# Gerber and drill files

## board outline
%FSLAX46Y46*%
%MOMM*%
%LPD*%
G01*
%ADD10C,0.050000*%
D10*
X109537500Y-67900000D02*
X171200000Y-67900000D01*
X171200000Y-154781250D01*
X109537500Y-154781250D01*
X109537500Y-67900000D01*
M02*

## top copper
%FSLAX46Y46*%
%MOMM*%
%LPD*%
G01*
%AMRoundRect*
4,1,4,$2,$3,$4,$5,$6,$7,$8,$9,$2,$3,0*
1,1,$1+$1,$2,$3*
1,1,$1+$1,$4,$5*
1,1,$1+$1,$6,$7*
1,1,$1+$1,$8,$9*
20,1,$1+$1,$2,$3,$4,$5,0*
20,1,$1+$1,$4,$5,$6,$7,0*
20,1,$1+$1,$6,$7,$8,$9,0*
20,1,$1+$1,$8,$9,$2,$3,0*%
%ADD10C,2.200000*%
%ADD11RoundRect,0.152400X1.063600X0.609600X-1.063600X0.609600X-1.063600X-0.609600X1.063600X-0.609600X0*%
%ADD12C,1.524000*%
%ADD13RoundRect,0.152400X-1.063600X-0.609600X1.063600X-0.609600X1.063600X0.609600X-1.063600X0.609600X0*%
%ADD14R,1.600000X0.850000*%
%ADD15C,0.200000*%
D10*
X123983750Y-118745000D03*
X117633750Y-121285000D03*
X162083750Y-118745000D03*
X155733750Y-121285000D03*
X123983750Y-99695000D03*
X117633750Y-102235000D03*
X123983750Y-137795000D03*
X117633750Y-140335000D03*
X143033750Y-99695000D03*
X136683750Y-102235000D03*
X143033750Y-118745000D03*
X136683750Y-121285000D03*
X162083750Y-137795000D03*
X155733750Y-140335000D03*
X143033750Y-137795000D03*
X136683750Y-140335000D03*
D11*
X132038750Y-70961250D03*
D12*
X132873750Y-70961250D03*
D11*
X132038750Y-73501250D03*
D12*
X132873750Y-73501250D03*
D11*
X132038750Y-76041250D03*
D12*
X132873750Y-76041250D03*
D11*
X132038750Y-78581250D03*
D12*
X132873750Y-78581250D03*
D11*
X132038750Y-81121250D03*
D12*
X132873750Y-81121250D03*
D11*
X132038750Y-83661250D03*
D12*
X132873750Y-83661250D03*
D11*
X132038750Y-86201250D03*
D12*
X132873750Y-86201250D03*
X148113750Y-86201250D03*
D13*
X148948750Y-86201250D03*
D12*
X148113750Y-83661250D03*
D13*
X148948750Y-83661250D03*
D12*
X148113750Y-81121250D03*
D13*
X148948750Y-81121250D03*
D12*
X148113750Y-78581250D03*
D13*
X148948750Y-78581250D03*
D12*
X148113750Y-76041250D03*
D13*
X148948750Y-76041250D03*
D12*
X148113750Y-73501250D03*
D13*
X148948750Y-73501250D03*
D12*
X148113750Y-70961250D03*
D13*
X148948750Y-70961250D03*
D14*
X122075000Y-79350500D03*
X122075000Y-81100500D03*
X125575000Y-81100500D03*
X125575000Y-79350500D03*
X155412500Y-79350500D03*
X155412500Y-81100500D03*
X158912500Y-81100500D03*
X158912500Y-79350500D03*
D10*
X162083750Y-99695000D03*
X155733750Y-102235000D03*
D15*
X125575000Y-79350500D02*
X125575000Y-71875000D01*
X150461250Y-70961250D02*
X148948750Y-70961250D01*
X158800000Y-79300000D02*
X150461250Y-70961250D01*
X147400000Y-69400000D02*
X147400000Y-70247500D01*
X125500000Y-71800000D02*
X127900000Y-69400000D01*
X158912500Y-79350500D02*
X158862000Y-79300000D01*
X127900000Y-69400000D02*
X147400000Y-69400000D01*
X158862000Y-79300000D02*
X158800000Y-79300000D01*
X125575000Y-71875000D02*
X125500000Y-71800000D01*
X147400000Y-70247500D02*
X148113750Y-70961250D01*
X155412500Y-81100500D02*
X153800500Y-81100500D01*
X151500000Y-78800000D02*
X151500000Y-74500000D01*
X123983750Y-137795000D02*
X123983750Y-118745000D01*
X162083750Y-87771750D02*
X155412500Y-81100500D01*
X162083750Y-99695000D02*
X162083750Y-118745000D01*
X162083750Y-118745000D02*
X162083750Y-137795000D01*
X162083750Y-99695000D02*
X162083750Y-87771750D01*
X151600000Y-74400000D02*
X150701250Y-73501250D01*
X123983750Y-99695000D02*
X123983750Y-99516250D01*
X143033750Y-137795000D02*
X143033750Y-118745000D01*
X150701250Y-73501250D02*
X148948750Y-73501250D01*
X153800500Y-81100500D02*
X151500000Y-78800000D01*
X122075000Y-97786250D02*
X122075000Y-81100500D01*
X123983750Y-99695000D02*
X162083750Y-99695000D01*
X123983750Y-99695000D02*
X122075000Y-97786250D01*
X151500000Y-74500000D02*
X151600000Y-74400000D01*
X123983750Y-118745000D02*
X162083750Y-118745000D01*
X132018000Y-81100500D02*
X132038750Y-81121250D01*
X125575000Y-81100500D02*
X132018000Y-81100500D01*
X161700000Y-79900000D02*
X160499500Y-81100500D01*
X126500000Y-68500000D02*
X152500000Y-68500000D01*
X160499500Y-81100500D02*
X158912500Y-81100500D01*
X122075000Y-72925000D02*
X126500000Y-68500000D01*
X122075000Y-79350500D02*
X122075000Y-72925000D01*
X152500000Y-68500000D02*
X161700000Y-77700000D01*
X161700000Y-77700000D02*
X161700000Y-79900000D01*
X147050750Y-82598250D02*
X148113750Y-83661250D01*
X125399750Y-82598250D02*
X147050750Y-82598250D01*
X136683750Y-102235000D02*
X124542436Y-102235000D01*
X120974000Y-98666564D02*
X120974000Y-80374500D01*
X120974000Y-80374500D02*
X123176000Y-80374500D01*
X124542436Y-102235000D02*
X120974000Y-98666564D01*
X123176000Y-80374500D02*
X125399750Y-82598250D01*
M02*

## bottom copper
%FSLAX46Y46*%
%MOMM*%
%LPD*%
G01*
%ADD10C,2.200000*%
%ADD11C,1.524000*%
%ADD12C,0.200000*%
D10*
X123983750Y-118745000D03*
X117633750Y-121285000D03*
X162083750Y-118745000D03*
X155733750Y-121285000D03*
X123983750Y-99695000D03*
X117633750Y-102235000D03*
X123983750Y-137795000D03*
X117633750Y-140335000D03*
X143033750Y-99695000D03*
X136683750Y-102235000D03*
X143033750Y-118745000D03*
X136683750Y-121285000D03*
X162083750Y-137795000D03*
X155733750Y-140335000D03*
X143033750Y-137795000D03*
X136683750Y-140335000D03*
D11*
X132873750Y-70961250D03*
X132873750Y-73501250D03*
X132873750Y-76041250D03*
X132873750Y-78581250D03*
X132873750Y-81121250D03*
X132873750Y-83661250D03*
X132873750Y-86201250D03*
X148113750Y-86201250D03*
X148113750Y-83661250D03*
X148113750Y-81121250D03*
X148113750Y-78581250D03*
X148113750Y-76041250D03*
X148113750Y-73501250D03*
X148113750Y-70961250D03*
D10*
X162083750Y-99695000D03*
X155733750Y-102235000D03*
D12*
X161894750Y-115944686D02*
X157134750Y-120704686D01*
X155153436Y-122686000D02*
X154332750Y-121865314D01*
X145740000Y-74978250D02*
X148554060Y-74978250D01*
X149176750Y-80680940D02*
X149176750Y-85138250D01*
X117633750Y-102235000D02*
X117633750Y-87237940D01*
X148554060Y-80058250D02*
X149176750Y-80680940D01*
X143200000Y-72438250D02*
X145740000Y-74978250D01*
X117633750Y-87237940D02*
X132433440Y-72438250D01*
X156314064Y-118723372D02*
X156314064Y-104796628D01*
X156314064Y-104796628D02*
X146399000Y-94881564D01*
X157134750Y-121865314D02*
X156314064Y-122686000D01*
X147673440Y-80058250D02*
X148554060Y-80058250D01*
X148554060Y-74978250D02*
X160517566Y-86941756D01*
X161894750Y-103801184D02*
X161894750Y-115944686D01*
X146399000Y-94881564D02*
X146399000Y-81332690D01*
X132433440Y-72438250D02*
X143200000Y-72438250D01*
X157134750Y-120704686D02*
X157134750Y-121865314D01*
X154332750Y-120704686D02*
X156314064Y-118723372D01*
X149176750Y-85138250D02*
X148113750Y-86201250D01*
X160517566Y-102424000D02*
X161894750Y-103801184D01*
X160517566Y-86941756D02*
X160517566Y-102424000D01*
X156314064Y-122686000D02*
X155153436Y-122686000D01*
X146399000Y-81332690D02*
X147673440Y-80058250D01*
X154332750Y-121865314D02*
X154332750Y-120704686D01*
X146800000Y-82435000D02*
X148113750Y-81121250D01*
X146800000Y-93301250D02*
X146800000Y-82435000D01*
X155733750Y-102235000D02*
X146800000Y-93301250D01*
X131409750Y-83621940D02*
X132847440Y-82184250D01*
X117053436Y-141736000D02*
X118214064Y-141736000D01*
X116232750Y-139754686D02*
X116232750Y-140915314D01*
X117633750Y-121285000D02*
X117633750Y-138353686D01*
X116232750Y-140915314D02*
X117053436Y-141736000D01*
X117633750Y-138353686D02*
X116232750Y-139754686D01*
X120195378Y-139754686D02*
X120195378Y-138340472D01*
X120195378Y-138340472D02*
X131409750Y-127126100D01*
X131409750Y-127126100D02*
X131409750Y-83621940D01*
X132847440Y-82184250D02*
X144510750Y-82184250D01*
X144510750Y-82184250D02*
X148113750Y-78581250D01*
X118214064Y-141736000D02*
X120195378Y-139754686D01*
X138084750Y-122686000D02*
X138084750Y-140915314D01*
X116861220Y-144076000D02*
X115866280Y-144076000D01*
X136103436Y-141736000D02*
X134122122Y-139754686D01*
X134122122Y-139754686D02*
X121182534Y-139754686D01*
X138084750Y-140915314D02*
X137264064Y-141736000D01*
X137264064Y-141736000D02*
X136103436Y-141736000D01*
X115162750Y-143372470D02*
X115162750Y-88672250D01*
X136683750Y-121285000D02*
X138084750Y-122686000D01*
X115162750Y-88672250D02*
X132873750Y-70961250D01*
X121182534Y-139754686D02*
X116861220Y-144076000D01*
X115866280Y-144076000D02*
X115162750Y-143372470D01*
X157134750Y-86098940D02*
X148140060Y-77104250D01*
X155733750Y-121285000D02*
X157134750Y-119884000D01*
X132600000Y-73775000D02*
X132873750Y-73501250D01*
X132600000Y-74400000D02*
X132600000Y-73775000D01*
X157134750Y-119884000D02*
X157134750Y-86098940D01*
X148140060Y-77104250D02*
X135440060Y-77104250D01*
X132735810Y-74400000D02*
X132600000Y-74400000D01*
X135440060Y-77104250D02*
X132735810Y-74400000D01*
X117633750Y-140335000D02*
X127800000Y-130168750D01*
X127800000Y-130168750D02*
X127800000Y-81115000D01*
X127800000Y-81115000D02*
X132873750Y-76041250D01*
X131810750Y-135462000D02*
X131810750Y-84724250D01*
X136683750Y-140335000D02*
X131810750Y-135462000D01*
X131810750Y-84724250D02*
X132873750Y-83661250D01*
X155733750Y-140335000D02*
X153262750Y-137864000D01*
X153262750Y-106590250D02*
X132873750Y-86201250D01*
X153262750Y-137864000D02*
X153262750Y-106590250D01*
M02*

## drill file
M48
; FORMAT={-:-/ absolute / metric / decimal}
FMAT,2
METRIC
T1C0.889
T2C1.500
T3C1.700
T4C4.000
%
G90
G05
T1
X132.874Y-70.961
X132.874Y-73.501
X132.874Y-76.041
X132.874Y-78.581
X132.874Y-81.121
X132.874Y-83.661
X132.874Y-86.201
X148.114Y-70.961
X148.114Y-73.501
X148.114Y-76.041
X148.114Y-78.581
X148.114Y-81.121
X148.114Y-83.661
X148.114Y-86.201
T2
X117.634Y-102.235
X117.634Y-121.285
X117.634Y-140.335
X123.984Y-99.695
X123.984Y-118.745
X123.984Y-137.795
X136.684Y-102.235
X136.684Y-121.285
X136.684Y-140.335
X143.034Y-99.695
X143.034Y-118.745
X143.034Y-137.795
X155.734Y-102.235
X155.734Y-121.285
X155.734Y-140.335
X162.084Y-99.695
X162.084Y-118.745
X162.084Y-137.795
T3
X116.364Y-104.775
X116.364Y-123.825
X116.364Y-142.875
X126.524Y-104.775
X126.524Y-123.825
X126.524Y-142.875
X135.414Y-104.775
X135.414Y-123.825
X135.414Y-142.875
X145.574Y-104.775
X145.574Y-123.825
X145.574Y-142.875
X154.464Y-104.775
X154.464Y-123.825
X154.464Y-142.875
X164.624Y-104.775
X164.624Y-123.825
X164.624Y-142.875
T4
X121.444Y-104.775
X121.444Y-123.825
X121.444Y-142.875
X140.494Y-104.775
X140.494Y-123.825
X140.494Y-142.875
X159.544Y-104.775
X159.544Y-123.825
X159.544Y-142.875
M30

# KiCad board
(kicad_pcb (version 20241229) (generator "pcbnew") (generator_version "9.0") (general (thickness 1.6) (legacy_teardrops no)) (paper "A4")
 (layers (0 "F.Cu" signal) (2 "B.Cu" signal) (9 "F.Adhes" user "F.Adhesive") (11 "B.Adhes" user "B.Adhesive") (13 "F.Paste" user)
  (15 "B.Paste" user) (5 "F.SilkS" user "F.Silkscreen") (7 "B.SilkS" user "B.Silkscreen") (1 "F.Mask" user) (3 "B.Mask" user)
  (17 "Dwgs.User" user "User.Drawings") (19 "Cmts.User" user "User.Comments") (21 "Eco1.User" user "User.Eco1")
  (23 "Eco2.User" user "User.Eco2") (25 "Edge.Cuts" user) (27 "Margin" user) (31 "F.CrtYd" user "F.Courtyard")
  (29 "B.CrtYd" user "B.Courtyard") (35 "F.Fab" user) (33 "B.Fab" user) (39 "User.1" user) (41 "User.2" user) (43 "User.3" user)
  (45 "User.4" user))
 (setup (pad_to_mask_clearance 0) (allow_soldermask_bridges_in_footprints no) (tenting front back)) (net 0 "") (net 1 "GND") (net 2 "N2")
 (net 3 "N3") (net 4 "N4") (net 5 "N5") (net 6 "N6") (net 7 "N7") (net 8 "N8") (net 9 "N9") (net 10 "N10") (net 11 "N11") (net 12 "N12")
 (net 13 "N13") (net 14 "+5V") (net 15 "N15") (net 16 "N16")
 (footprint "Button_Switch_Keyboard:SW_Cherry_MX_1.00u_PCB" (layer "F.Cu") (at 123.98375 118.745)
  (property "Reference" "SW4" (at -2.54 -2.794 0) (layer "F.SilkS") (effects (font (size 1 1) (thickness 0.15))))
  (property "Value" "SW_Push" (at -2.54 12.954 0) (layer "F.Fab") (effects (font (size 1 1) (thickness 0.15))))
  (pad "" np_thru_hole circle (at -7.62 5.08) (size 1.7 1.7) (drill 1.7) (layers "*.Cu" "*.Mask"))
  (pad "" np_thru_hole circle (at -2.54 5.08) (size 4 4) (drill 4) (layers "*.Cu" "*.Mask"))
  (pad "" np_thru_hole circle (at 2.54 5.08) (size 1.7 1.7) (drill 1.7) (layers "*.Cu" "*.Mask"))
  (pad "1" thru_hole circle (at 0 0) (size 2.2 2.2) (drill 1.5) (layers "*.Cu" "*.Mask") (remove_unused_layers no) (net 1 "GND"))
  (pad "2" thru_hole circle (at -6.35 2.54) (size 2.2 2.2) (drill 1.5) (layers "*.Cu" "*.Mask") (remove_unused_layers no) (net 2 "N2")))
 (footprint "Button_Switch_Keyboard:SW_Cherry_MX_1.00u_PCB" (layer "F.Cu") (at 162.08375 118.745)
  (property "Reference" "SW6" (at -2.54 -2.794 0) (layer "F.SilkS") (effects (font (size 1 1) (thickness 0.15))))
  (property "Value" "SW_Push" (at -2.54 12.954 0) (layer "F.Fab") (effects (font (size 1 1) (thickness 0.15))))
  (pad "" np_thru_hole circle (at -7.62 5.08) (size 1.7 1.7) (drill 1.7) (layers "*.Cu" "*.Mask"))
  (pad "" np_thru_hole circle (at -2.54 5.08) (size 4 4) (drill 4) (layers "*.Cu" "*.Mask"))
  (pad "" np_thru_hole circle (at 2.54 5.08) (size 1.7 1.7) (drill 1.7) (layers "*.Cu" "*.Mask"))
  (pad "1" thru_hole circle (at 0 0) (size 2.2 2.2) (drill 1.5) (layers "*.Cu" "*.Mask") (remove_unused_layers no) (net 1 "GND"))
  (pad "2" thru_hole circle (at -6.35 2.54) (size 2.2 2.2) (drill 1.5) (layers "*.Cu" "*.Mask") (remove_unused_layers no) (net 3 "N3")))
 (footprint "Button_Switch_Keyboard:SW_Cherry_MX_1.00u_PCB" (layer "F.Cu") (at 123.98375 99.695)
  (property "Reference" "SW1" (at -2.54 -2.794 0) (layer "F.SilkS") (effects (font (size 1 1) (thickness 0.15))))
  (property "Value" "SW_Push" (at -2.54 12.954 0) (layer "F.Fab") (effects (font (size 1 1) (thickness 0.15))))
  (pad "" np_thru_hole circle (at -7.62 5.08) (size 1.7 1.7) (drill 1.7) (layers "*.Cu" "*.Mask"))
  (pad "" np_thru_hole circle (at -2.54 5.08) (size 4 4) (drill 4) (layers "*.Cu" "*.Mask"))
  (pad "" np_thru_hole circle (at 2.54 5.08) (size 1.7 1.7) (drill 1.7) (layers "*.Cu" "*.Mask"))
  (pad "1" thru_hole circle (at 0 0) (size 2.2 2.2) (drill 1.5) (layers "*.Cu" "*.Mask") (remove_unused_layers no) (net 1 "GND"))
  (pad "2" thru_hole circle (at -6.35 2.54) (size 2.2 2.2) (drill 1.5) (layers "*.Cu" "*.Mask") (remove_unused_layers no) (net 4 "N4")))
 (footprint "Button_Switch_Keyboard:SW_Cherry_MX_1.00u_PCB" (layer "F.Cu") (at 123.98375 137.795)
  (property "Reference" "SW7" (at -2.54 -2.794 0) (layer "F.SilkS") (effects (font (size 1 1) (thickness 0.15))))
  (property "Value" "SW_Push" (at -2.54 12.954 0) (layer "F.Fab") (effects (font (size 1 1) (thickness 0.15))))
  (pad "" np_thru_hole circle (at -7.62 5.08) (size 1.7 1.7) (drill 1.7) (layers "*.Cu" "*.Mask"))
  (pad "" np_thru_hole circle (at -2.54 5.08) (size 4 4) (drill 4) (layers "*.Cu" "*.Mask"))
  (pad "" np_thru_hole circle (at 2.54 5.08) (size 1.7 1.7) (drill 1.7) (layers "*.Cu" "*.Mask"))
  (pad "1" thru_hole circle (at 0 0) (size 2.2 2.2) (drill 1.5) (layers "*.Cu" "*.Mask") (remove_unused_layers no) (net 1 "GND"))
  (pad "2" thru_hole circle (at -6.35 2.54) (size 2.2 2.2) (drill 1.5) (layers "*.Cu" "*.Mask") (remove_unused_layers no) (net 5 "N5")))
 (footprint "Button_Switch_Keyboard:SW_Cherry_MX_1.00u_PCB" (layer "F.Cu") (at 143.03375 99.695)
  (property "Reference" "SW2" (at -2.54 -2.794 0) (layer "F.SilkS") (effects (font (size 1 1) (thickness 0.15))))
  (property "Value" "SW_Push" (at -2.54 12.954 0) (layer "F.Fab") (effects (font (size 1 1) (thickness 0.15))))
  (pad "" np_thru_hole circle (at -7.62 5.08) (size 1.7 1.7) (drill 1.7) (layers "*.Cu" "*.Mask"))
  (pad "" np_thru_hole circle (at -2.54 5.08) (size 4 4) (drill 4) (layers "*.Cu" "*.Mask"))
  (pad "" np_thru_hole circle (at 2.54 5.08) (size 1.7 1.7) (drill 1.7) (layers "*.Cu" "*.Mask"))
  (pad "1" thru_hole circle (at 0 0) (size 2.2 2.2) (drill 1.5) (layers "*.Cu" "*.Mask") (remove_unused_layers no) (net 1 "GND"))
  (pad "2" thru_hole circle (at -6.35 2.54) (size 2.2 2.2) (drill 1.5) (layers "*.Cu" "*.Mask") (remove_unused_layers no) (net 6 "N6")))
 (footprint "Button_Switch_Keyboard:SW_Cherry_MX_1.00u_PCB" (layer "F.Cu") (at 143.03375 118.745)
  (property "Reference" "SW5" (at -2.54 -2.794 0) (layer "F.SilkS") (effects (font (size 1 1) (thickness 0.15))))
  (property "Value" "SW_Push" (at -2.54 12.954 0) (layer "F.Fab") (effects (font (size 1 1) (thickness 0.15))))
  (pad "" np_thru_hole circle (at -7.62 5.08) (size 1.7 1.7) (drill 1.7) (layers "*.Cu" "*.Mask"))
  (pad "" np_thru_hole circle (at -2.54 5.08) (size 4 4) (drill 4) (layers "*.Cu" "*.Mask"))
  (pad "" np_thru_hole circle (at 2.54 5.08) (size 1.7 1.7) (drill 1.7) (layers "*.Cu" "*.Mask"))
  (pad "1" thru_hole circle (at 0 0) (size 2.2 2.2) (drill 1.5) (layers "*.Cu" "*.Mask") (remove_unused_layers no) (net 1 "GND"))
  (pad "2" thru_hole circle (at -6.35 2.54) (size 2.2 2.2) (drill 1.5) (layers "*.Cu" "*.Mask") (remove_unused_layers no) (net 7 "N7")))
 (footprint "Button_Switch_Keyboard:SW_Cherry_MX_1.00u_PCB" (layer "F.Cu") (at 162.08375 137.795)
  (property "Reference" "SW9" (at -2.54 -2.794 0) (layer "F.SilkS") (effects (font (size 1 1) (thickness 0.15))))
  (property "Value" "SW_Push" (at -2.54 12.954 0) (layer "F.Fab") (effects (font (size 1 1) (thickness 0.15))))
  (pad "" np_thru_hole circle (at -7.62 5.08) (size 1.7 1.7) (drill 1.7) (layers "*.Cu" "*.Mask"))
  (pad "" np_thru_hole circle (at -2.54 5.08) (size 4 4) (drill 4) (layers "*.Cu" "*.Mask"))
  (pad "" np_thru_hole circle (at 2.54 5.08) (size 1.7 1.7) (drill 1.7) (layers "*.Cu" "*.Mask"))
  (pad "1" thru_hole circle (at 0 0) (size 2.2 2.2) (drill 1.5) (layers "*.Cu" "*.Mask") (remove_unused_layers no) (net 1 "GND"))
  (pad "2" thru_hole circle (at -6.35 2.54) (size 2.2 2.2) (drill 1.5) (layers "*.Cu" "*.Mask") (remove_unused_layers no) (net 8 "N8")))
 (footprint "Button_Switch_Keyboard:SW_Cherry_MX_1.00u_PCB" (layer "F.Cu") (at 143.03375 137.795)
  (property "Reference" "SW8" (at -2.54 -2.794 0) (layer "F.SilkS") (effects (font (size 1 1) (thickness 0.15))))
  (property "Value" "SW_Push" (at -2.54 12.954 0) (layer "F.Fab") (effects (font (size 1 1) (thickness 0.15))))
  (pad "" np_thru_hole circle (at -7.62 5.08) (size 1.7 1.7) (drill 1.7) (layers "*.Cu" "*.Mask"))
  (pad "" np_thru_hole circle (at -2.54 5.08) (size 4 4) (drill 4) (layers "*.Cu" "*.Mask"))
  (pad "" np_thru_hole circle (at 2.54 5.08) (size 1.7 1.7) (drill 1.7) (layers "*.Cu" "*.Mask"))
  (pad "1" thru_hole circle (at 0 0) (size 2.2 2.2) (drill 1.5) (layers "*.Cu" "*.Mask") (remove_unused_layers no) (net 1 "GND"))
  (pad "2" thru_hole circle (at -6.35 2.54) (size 2.2 2.2) (drill 1.5) (layers "*.Cu" "*.Mask") (remove_unused_layers no) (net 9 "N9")))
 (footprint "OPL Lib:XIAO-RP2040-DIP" (layer "F.Cu") (at 140.49375 78.58125)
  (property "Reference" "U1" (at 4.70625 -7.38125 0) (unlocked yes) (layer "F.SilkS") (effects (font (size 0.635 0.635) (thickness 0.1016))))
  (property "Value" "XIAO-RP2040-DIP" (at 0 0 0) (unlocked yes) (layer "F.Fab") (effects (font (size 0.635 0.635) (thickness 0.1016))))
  (pad "1" smd roundrect (at -8.455 -7.62 180) (size 2.432 1.524) (layers "F.Cu" "F.Mask") (roundrect_rratio 0.1) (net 7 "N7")
   (thermal_bridge_angle 45))
  (pad "1" thru_hole circle (at -7.62 -7.62 180) (size 1.524 1.524) (drill 0.889) (layers "*.Cu" "*.Mask") (remove_unused_layers no)
   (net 7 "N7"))
  (pad "2" smd roundrect (at -8.455 -5.08 180) (size 2.432 1.524) (layers "F.Cu" "F.Mask") (roundrect_rratio 0.1) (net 3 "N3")
   (thermal_bridge_angle 45))
  (pad "2" thru_hole circle (at -7.62 -5.08 180) (size 1.524 1.524) (drill 0.889) (layers "*.Cu" "*.Mask") (remove_unused_layers no)
   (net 3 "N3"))
  (pad "3" smd roundrect (at -8.455 -2.54 180) (size 2.432 1.524) (layers "F.Cu" "F.Mask") (roundrect_rratio 0.1) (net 5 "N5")
   (thermal_bridge_angle 45))
  (pad "3" thru_hole circle (at -7.62 -2.54 180) (size 1.524 1.524) (drill 0.889) (layers "*.Cu" "*.Mask") (remove_unused_layers no)
   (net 5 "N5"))
  (pad "4" smd roundrect (at -8.455 0 180) (size 2.432 1.524) (layers "F.Cu" "F.Mask") (roundrect_rratio 0.1) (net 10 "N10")
   (thermal_bridge_angle 45))
  (pad "4" thru_hole circle (at -7.62 0 180) (size 1.524 1.524) (drill 0.889) (layers "*.Cu" "*.Mask") (remove_unused_layers no)
   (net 10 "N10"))
  (pad "5" smd roundrect (at -8.455 2.54 180) (size 2.432 1.524) (layers "F.Cu" "F.Mask") (roundrect_rratio 0.1) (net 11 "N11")
   (thermal_bridge_angle 45))
  (pad "5" thru_hole circle (at -7.62 2.54 180) (size 1.524 1.524) (drill 0.889) (layers "*.Cu" "*.Mask") (remove_unused_layers no)
   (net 11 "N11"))
  (pad "6" smd roundrect (at -8.455 5.08 180) (size 2.432 1.524) (layers "F.Cu" "F.Mask") (roundrect_rratio 0.1) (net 9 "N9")
   (thermal_bridge_angle 45))
  (pad "6" thru_hole circle (at -7.62 5.08 180) (size 1.524 1.524) (drill 0.889) (layers "*.Cu" "*.Mask") (remove_unused_layers no)
   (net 9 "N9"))
  (pad "7" smd roundrect (at -8.455 7.62 180) (size 2.432 1.524) (layers "F.Cu" "F.Mask") (roundrect_rratio 0.1) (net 8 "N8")
   (thermal_bridge_angle 45))
  (pad "7" thru_hole circle (at -7.62 7.62 180) (size 1.524 1.524) (drill 0.889) (layers "*.Cu" "*.Mask") (remove_unused_layers no)
   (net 8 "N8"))
  (pad "8" thru_hole circle (at 7.62 7.62) (size 1.524 1.524) (drill 0.889) (layers "*.Cu" "*.Mask") (remove_unused_layers no) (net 4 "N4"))
  (pad "8" smd roundrect (at 8.455 7.62) (size 2.432 1.524) (layers "F.Cu" "F.Mask") (roundrect_rratio 0.1) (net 4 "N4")
   (thermal_bridge_angle 45))
  (pad "9" thru_hole circle (at 7.62 5.08) (size 1.524 1.524) (drill 0.889) (layers "*.Cu" "*.Mask") (remove_unused_layers no) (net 6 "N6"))
  (pad "9" smd roundrect (at 8.455 5.08) (size 2.432 1.524) (layers "F.Cu" "F.Mask") (roundrect_rratio 0.1) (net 6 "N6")
   (thermal_bridge_angle 45))
  (pad "10" thru_hole circle (at 7.62 2.54) (size 1.524 1.524) (drill 0.889) (layers "*.Cu" "*.Mask") (remove_unused_layers no)
   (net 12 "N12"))
  (pad "10" smd roundrect (at 8.455 2.54) (size 2.432 1.524) (layers "F.Cu" "F.Mask") (roundrect_rratio 0.1) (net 12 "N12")
   (thermal_bridge_angle 45))
  (pad "11" thru_hole circle (at 7.62 0) (size 1.524 1.524) (drill 0.889) (layers "*.Cu" "*.Mask") (remove_unused_layers no) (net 2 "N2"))
  (pad "11" smd roundrect (at 8.455 0) (size 2.432 1.524) (layers "F.Cu" "F.Mask") (roundrect_rratio 0.1) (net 2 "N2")
   (thermal_bridge_angle 45))
  (pad "12" thru_hole circle (at 7.62 -2.54) (size 1.524 1.524) (drill 0.889) (layers "*.Cu" "*.Mask") (remove_unused_layers no)
   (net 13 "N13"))
  (pad "12" smd roundrect (at 8.455 -2.54) (size 2.432 1.524) (layers "F.Cu" "F.Mask") (roundrect_rratio 0.1) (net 13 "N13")
   (thermal_bridge_angle 45))
  (pad "13" thru_hole circle (at 7.62 -5.08) (size 1.524 1.524) (drill 0.889) (layers "*.Cu" "*.Mask") (remove_unused_layers no)
   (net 1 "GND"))
  (pad "13" smd roundrect (at 8.455 -5.08) (size 2.432 1.524) (layers "F.Cu" "F.Mask") (roundrect_rratio 0.1) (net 1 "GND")
   (thermal_bridge_angle 45))
  (pad "14" thru_hole circle (at 7.62 -7.62) (size 1.524 1.524) (drill 0.889) (layers "*.Cu" "*.Mask") (remove_unused_layers no)
   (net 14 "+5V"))
  (pad "14" smd roundrect (at 8.455 -7.62) (size 2.432 1.524) (layers "F.Cu" "F.Mask") (roundrect_rratio 0.1) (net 14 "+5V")
   (thermal_bridge_angle 45)))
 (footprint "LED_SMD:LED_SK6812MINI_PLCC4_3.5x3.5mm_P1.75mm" (layer "F.Cu") (at 123.825 80.2255)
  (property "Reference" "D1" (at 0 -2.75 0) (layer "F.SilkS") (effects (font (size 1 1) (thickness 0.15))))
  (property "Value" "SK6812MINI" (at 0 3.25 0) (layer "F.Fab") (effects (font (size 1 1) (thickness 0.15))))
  (pad "1" smd rect (at -1.75 -0.875) (size 1.6 0.85) (layers "F.Cu" "F.Mask" "F.Paste") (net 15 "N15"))
  (pad "2" smd rect (at -1.75 0.875) (size 1.6 0.85) (layers "F.Cu" "F.Mask" "F.Paste") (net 1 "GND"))
  (pad "3" smd rect (at 1.75 0.875) (size 1.6 0.85) (layers "F.Cu" "F.Mask" "F.Paste") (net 11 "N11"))
  (pad "4" smd rect (at 1.75 -0.875) (size 1.6 0.85) (layers "F.Cu" "F.Mask" "F.Paste") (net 14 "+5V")))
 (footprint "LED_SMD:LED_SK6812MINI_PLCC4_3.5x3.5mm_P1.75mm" (layer "F.Cu") (at 157.1625 80.2255)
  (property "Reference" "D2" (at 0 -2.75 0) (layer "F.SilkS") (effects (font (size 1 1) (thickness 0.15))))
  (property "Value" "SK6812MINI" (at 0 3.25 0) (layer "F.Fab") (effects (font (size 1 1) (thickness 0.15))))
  (pad "1" smd rect (at -1.75 -0.875) (size 1.6 0.85) (layers "F.Cu" "F.Mask" "F.Paste") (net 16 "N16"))
  (pad "2" smd rect (at -1.75 0.875) (size 1.6 0.85) (layers "F.Cu" "F.Mask" "F.Paste") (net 1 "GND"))
  (pad "3" smd rect (at 1.75 0.875) (size 1.6 0.85) (layers "F.Cu" "F.Mask" "F.Paste") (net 15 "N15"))
  (pad "4" smd rect (at 1.75 -0.875) (size 1.6 0.85) (layers "F.Cu" "F.Mask" "F.Paste") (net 14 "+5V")))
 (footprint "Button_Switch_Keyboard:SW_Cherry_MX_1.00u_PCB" (layer "F.Cu") (at 162.08375 99.695)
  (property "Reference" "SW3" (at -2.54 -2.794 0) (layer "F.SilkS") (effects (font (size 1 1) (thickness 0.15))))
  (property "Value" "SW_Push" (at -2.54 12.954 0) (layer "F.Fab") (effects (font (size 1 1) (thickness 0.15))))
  (pad "" np_thru_hole circle (at -7.62 5.08) (size 1.7 1.7) (drill 1.7) (layers "*.Cu" "*.Mask"))
  (pad "" np_thru_hole circle (at -2.54 5.08) (size 4 4) (drill 4) (layers "*.Cu" "*.Mask"))
  (pad "" np_thru_hole circle (at 2.54 5.08) (size 1.7 1.7) (drill 1.7) (layers "*.Cu" "*.Mask"))
  (pad "1" thru_hole circle (at 0 0) (size 2.2 2.2) (drill 1.5) (layers "*.Cu" "*.Mask") (remove_unused_layers no) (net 1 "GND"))
  (pad "2" thru_hole circle (at -6.35 2.54) (size 2.2 2.2) (drill 1.5) (layers "*.Cu" "*.Mask") (remove_unused_layers no) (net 12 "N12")))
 (gr_rect (start 109.5375 67.9) (end 171.2 154.78125) (stroke (width 0.05) (type default)) (fill no) (layer "Edge.Cuts"))
 (segment (start 125.575 79.3505) (end 125.575 71.875) (width 0.2) (layer "F.Cu") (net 14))
 (segment (start 150.46125 70.96125) (end 148.94875 70.96125) (width 0.2) (layer "F.Cu") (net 14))
 (segment (start 158.8 79.3) (end 150.46125 70.96125) (width 0.2) (layer "F.Cu") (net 14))
 (segment (start 147.4 69.4) (end 147.4 70.2475) (width 0.2) (layer "F.Cu") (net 14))
 (segment (start 125.5 71.8) (end 127.9 69.4) (width 0.2) (layer "F.Cu") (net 14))
 (segment (start 158.9125 79.3505) (end 158.862 79.3) (width 0.2) (layer "F.Cu") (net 14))
 (segment (start 127.9 69.4) (end 147.4 69.4) (width 0.2) (layer "F.Cu") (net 14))
 (segment (start 158.862 79.3) (end 158.8 79.3) (width 0.2) (layer "F.Cu") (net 14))
 (segment (start 125.575 71.875) (end 125.5 71.8) (width 0.2) (layer "F.Cu") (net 14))
 (segment (start 147.4 70.2475) (end 148.11375 70.96125) (width 0.2) (layer "F.Cu") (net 14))
 (segment (start 155.4125 81.1005) (end 153.8005 81.1005) (width 0.2) (layer "F.Cu") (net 1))
 (segment (start 151.5 78.8) (end 151.5 74.5) (width 0.2) (layer "F.Cu") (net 1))
 (segment (start 123.98375 137.795) (end 123.98375 118.745) (width 0.2) (layer "F.Cu") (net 1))
 (segment (start 162.08375 87.77175) (end 155.4125 81.1005) (width 0.2) (layer "F.Cu") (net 1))
 (segment (start 162.08375 99.695) (end 162.08375 118.745) (width 0.2) (layer "F.Cu") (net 1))
 (segment (start 162.08375 118.745) (end 162.08375 137.795) (width 0.2) (layer "F.Cu") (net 1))
 (segment (start 162.08375 99.695) (end 162.08375 87.77175) (width 0.2) (layer "F.Cu") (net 1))
 (segment (start 151.6 74.4) (end 150.70125 73.50125) (width 0.2) (layer "F.Cu") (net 1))
 (segment (start 123.98375 99.695) (end 123.98375 99.51625) (width 0.2) (layer "F.Cu") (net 1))
 (segment (start 143.03375 137.795) (end 143.03375 118.745) (width 0.2) (layer "F.Cu") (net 1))
 (segment (start 150.70125 73.50125) (end 148.94875 73.50125) (width 0.2) (layer "F.Cu") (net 1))
 (segment (start 153.8005 81.1005) (end 151.5 78.8) (width 0.2) (layer "F.Cu") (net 1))
 (segment (start 122.075 97.78625) (end 122.075 81.1005) (width 0.2) (layer "F.Cu") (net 1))
 (segment (start 123.98375 99.695) (end 162.08375 99.695) (width 0.2) (layer "F.Cu") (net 1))
 (segment (start 123.98375 99.695) (end 122.075 97.78625) (width 0.2) (layer "F.Cu") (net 1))
 (segment (start 151.5 74.5) (end 151.6 74.4) (width 0.2) (layer "F.Cu") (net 1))
 (segment (start 123.98375 118.745) (end 162.08375 118.745) (width 0.2) (layer "F.Cu") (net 1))
 (segment (start 132.018 81.1005) (end 132.03875 81.12125) (width 0.2) (layer "F.Cu") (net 11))
 (segment (start 125.575 81.1005) (end 132.018 81.1005) (width 0.2) (layer "F.Cu") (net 11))
 (segment (start 161.7 79.9) (end 160.4995 81.1005) (width 0.2) (layer "F.Cu") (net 15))
 (segment (start 126.5 68.5) (end 152.5 68.5) (width 0.2) (layer "F.Cu") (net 15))
 (segment (start 160.4995 81.1005) (end 158.9125 81.1005) (width 0.2) (layer "F.Cu") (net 15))
 (segment (start 122.075 72.925) (end 126.5 68.5) (width 0.2) (layer "F.Cu") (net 15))
 (segment (start 122.075 79.3505) (end 122.075 72.925) (width 0.2) (layer "F.Cu") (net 15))
 (segment (start 152.5 68.5) (end 161.7 77.7) (width 0.2) (layer "F.Cu") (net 15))
 (segment (start 161.7 77.7) (end 161.7 79.9) (width 0.2) (layer "F.Cu") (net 15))
 (segment (start 161.89475 115.944686) (end 157.13475 120.704686) (width 0.2) (layer "B.Cu") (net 4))
 (segment (start 155.153436 122.686) (end 154.33275 121.865314) (width 0.2) (layer "B.Cu") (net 4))
 (segment (start 145.74 74.97825) (end 148.55406 74.97825) (width 0.2) (layer "B.Cu") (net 4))
 (segment (start 149.17675 80.68094) (end 149.17675 85.13825) (width 0.2) (layer "B.Cu") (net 4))
 (segment (start 117.63375 102.235) (end 117.63375 87.23794) (width 0.2) (layer "B.Cu") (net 4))
 (segment (start 148.55406 80.05825) (end 149.17675 80.68094) (width 0.2) (layer "B.Cu") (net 4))
 (segment (start 143.2 72.43825) (end 145.74 74.97825) (width 0.2) (layer "B.Cu") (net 4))
 (segment (start 117.63375 87.23794) (end 132.43344 72.43825) (width 0.2) (layer "B.Cu") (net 4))
 (segment (start 156.314064 118.723372) (end 156.314064 104.796628) (width 0.2) (layer "B.Cu") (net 4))
 (segment (start 156.314064 104.796628) (end 146.399 94.881564) (width 0.2) (layer "B.Cu") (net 4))
 (segment (start 157.13475 121.865314) (end 156.314064 122.686) (width 0.2) (layer "B.Cu") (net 4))
 (segment (start 147.67344 80.05825) (end 148.55406 80.05825) (width 0.2) (layer "B.Cu") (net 4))
 (segment (start 148.55406 74.97825) (end 160.517566 86.941756) (width 0.2) (layer "B.Cu") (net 4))
 (segment (start 161.89475 103.801184) (end 161.89475 115.944686) (width 0.2) (layer "B.Cu") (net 4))
 (segment (start 146.399 94.881564) (end 146.399 81.33269) (width 0.2) (layer "B.Cu") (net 4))
 (segment (start 132.43344 72.43825) (end 143.2 72.43825) (width 0.2) (layer "B.Cu") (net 4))
 (segment (start 157.13475 120.704686) (end 157.13475 121.865314) (width 0.2) (layer "B.Cu") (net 4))
 (segment (start 154.33275 120.704686) (end 156.314064 118.723372) (width 0.2) (layer "B.Cu") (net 4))
 (segment (start 149.17675 85.13825) (end 148.11375 86.20125) (width 0.2) (layer "B.Cu") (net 4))
 (segment (start 160.517566 102.424) (end 161.89475 103.801184) (width 0.2) (layer "B.Cu") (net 4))
 (segment (start 160.517566 86.941756) (end 160.517566 102.424) (width 0.2) (layer "B.Cu") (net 4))
 (segment (start 156.314064 122.686) (end 155.153436 122.686) (width 0.2) (layer "B.Cu") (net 4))
 (segment (start 146.399 81.33269) (end 147.67344 80.05825) (width 0.2) (layer "B.Cu") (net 4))
 (segment (start 154.33275 121.865314) (end 154.33275 120.704686) (width 0.2) (layer "B.Cu") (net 4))
 (segment (start 147.05075 82.59825) (end 148.11375 83.66125) (width 0.2) (layer "F.Cu") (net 6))
 (segment (start 125.39975 82.59825) (end 147.05075 82.59825) (width 0.2) (layer "F.Cu") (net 6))
 (segment (start 136.68375 102.235) (end 124.542436 102.235) (width 0.2) (layer "F.Cu") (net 6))
 (segment (start 120.974 98.666564) (end 120.974 80.3745) (width 0.2) (layer "F.Cu") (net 6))
 (segment (start 120.974 80.3745) (end 123.176 80.3745) (width 0.2) (layer "F.Cu") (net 6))
 (segment (start 124.542436 102.235) (end 120.974 98.666564) (width 0.2) (layer "F.Cu") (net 6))
 (segment (start 123.176 80.3745) (end 125.39975 82.59825) (width 0.2) (layer "F.Cu") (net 6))
 (segment (start 146.8 82.435) (end 148.11375 81.12125) (width 0.2) (layer "B.Cu") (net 12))
 (segment (start 146.8 93.30125) (end 146.8 82.435) (width 0.2) (layer "B.Cu") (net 12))
 (segment (start 155.73375 102.235) (end 146.8 93.30125) (width 0.2) (layer "B.Cu") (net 12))
 (segment (start 131.40975 83.62194) (end 132.84744 82.18425) (width 0.2) (layer "B.Cu") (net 2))
 (segment (start 117.053436 141.736) (end 118.214064 141.736) (width 0.2) (layer "B.Cu") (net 2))
 (segment (start 116.23275 139.754686) (end 116.23275 140.915314) (width 0.2) (layer "B.Cu") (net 2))
 (segment (start 117.63375 121.285) (end 117.63375 138.353686) (width 0.2) (layer "B.Cu") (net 2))
 (segment (start 116.23275 140.915314) (end 117.053436 141.736) (width 0.2) (layer "B.Cu") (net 2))
 (segment (start 117.63375 138.353686) (end 116.23275 139.754686) (width 0.2) (layer "B.Cu") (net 2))
 (segment (start 120.195378 139.754686) (end 120.195378 138.340472) (width 0.2) (layer "B.Cu") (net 2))
 (segment (start 120.195378 138.340472) (end 131.40975 127.1261) (width 0.2) (layer "B.Cu") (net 2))
 (segment (start 131.40975 127.1261) (end 131.40975 83.62194) (width 0.2) (layer "B.Cu") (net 2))
 (segment (start 132.84744 82.18425) (end 144.51075 82.18425) (width 0.2) (layer "B.Cu") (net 2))
 (segment (start 144.51075 82.18425) (end 148.11375 78.58125) (width 0.2) (layer "B.Cu") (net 2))
 (segment (start 118.214064 141.736) (end 120.195378 139.754686) (width 0.2) (layer "B.Cu") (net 2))
 (segment (start 138.08475 122.686) (end 138.08475 140.915314) (width 0.2) (layer "B.Cu") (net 7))
 (segment (start 116.86122 144.076) (end 115.86628 144.076) (width 0.2) (layer "B.Cu") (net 7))
 (segment (start 136.103436 141.736) (end 134.122122 139.754686) (width 0.2) (layer "B.Cu") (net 7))
 (segment (start 134.122122 139.754686) (end 121.182534 139.754686) (width 0.2) (layer "B.Cu") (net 7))
 (segment (start 138.08475 140.915314) (end 137.264064 141.736) (width 0.2) (layer "B.Cu") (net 7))
 (segment (start 137.264064 141.736) (end 136.103436 141.736) (width 0.2) (layer "B.Cu") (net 7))
 (segment (start 115.16275 143.37247) (end 115.16275 88.67225) (width 0.2) (layer "B.Cu") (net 7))
 (segment (start 136.68375 121.285) (end 138.08475 122.686) (width 0.2) (layer "B.Cu") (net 7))
 (segment (start 115.16275 88.67225) (end 132.87375 70.96125) (width 0.2) (layer "B.Cu") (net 7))
 (segment (start 121.182534 139.754686) (end 116.86122 144.076) (width 0.2) (layer "B.Cu") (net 7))
 (segment (start 115.86628 144.076) (end 115.16275 143.37247) (width 0.2) (layer "B.Cu") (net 7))
 (segment (start 157.13475 86.09894) (end 148.14006 77.10425) (width 0.2) (layer "B.Cu") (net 3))
 (segment (start 155.73375 121.285) (end 157.13475 119.884) (width 0.2) (layer "B.Cu") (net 3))
 (segment (start 132.6 73.775) (end 132.87375 73.50125) (width 0.2) (layer "B.Cu") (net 3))
 (segment (start 132.6 74.4) (end 132.6 73.775) (width 0.2) (layer "B.Cu") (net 3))
 (segment (start 157.13475 119.884) (end 157.13475 86.09894) (width 0.2) (layer "B.Cu") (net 3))
 (segment (start 148.14006 77.10425) (end 135.44006 77.10425) (width 0.2) (layer "B.Cu") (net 3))
 (segment (start 132.73581 74.4) (end 132.6 74.4) (width 0.2) (layer "B.Cu") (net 3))
 (segment (start 135.44006 77.10425) (end 132.73581 74.4) (width 0.2) (layer "B.Cu") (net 3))
 (segment (start 117.63375 140.335) (end 127.8 130.16875) (width 0.2) (layer "B.Cu") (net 5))
 (segment (start 127.8 130.16875) (end 127.8 81.115) (width 0.2) (layer "B.Cu") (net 5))
 (segment (start 127.8 81.115) (end 132.87375 76.04125) (width 0.2) (layer "B.Cu") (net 5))
 (segment (start 131.81075 135.462) (end 131.81075 84.72425) (width 0.2) (layer "B.Cu") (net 9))
 (segment (start 136.68375 140.335) (end 131.81075 135.462) (width 0.2) (layer "B.Cu") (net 9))
 (segment (start 131.81075 84.72425) (end 132.87375 83.66125) (width 0.2) (layer "B.Cu") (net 9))
 (segment (start 155.73375 140.335) (end 153.26275 137.864) (width 0.2) (layer "B.Cu") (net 8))
 (segment (start 153.26275 106.59025) (end 132.87375 86.20125) (width 0.2) (layer "B.Cu") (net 8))
 (segment (start 153.26275 137.864) (end 153.26275 106.59025) (width 0.2) (layer "B.Cu") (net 8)))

